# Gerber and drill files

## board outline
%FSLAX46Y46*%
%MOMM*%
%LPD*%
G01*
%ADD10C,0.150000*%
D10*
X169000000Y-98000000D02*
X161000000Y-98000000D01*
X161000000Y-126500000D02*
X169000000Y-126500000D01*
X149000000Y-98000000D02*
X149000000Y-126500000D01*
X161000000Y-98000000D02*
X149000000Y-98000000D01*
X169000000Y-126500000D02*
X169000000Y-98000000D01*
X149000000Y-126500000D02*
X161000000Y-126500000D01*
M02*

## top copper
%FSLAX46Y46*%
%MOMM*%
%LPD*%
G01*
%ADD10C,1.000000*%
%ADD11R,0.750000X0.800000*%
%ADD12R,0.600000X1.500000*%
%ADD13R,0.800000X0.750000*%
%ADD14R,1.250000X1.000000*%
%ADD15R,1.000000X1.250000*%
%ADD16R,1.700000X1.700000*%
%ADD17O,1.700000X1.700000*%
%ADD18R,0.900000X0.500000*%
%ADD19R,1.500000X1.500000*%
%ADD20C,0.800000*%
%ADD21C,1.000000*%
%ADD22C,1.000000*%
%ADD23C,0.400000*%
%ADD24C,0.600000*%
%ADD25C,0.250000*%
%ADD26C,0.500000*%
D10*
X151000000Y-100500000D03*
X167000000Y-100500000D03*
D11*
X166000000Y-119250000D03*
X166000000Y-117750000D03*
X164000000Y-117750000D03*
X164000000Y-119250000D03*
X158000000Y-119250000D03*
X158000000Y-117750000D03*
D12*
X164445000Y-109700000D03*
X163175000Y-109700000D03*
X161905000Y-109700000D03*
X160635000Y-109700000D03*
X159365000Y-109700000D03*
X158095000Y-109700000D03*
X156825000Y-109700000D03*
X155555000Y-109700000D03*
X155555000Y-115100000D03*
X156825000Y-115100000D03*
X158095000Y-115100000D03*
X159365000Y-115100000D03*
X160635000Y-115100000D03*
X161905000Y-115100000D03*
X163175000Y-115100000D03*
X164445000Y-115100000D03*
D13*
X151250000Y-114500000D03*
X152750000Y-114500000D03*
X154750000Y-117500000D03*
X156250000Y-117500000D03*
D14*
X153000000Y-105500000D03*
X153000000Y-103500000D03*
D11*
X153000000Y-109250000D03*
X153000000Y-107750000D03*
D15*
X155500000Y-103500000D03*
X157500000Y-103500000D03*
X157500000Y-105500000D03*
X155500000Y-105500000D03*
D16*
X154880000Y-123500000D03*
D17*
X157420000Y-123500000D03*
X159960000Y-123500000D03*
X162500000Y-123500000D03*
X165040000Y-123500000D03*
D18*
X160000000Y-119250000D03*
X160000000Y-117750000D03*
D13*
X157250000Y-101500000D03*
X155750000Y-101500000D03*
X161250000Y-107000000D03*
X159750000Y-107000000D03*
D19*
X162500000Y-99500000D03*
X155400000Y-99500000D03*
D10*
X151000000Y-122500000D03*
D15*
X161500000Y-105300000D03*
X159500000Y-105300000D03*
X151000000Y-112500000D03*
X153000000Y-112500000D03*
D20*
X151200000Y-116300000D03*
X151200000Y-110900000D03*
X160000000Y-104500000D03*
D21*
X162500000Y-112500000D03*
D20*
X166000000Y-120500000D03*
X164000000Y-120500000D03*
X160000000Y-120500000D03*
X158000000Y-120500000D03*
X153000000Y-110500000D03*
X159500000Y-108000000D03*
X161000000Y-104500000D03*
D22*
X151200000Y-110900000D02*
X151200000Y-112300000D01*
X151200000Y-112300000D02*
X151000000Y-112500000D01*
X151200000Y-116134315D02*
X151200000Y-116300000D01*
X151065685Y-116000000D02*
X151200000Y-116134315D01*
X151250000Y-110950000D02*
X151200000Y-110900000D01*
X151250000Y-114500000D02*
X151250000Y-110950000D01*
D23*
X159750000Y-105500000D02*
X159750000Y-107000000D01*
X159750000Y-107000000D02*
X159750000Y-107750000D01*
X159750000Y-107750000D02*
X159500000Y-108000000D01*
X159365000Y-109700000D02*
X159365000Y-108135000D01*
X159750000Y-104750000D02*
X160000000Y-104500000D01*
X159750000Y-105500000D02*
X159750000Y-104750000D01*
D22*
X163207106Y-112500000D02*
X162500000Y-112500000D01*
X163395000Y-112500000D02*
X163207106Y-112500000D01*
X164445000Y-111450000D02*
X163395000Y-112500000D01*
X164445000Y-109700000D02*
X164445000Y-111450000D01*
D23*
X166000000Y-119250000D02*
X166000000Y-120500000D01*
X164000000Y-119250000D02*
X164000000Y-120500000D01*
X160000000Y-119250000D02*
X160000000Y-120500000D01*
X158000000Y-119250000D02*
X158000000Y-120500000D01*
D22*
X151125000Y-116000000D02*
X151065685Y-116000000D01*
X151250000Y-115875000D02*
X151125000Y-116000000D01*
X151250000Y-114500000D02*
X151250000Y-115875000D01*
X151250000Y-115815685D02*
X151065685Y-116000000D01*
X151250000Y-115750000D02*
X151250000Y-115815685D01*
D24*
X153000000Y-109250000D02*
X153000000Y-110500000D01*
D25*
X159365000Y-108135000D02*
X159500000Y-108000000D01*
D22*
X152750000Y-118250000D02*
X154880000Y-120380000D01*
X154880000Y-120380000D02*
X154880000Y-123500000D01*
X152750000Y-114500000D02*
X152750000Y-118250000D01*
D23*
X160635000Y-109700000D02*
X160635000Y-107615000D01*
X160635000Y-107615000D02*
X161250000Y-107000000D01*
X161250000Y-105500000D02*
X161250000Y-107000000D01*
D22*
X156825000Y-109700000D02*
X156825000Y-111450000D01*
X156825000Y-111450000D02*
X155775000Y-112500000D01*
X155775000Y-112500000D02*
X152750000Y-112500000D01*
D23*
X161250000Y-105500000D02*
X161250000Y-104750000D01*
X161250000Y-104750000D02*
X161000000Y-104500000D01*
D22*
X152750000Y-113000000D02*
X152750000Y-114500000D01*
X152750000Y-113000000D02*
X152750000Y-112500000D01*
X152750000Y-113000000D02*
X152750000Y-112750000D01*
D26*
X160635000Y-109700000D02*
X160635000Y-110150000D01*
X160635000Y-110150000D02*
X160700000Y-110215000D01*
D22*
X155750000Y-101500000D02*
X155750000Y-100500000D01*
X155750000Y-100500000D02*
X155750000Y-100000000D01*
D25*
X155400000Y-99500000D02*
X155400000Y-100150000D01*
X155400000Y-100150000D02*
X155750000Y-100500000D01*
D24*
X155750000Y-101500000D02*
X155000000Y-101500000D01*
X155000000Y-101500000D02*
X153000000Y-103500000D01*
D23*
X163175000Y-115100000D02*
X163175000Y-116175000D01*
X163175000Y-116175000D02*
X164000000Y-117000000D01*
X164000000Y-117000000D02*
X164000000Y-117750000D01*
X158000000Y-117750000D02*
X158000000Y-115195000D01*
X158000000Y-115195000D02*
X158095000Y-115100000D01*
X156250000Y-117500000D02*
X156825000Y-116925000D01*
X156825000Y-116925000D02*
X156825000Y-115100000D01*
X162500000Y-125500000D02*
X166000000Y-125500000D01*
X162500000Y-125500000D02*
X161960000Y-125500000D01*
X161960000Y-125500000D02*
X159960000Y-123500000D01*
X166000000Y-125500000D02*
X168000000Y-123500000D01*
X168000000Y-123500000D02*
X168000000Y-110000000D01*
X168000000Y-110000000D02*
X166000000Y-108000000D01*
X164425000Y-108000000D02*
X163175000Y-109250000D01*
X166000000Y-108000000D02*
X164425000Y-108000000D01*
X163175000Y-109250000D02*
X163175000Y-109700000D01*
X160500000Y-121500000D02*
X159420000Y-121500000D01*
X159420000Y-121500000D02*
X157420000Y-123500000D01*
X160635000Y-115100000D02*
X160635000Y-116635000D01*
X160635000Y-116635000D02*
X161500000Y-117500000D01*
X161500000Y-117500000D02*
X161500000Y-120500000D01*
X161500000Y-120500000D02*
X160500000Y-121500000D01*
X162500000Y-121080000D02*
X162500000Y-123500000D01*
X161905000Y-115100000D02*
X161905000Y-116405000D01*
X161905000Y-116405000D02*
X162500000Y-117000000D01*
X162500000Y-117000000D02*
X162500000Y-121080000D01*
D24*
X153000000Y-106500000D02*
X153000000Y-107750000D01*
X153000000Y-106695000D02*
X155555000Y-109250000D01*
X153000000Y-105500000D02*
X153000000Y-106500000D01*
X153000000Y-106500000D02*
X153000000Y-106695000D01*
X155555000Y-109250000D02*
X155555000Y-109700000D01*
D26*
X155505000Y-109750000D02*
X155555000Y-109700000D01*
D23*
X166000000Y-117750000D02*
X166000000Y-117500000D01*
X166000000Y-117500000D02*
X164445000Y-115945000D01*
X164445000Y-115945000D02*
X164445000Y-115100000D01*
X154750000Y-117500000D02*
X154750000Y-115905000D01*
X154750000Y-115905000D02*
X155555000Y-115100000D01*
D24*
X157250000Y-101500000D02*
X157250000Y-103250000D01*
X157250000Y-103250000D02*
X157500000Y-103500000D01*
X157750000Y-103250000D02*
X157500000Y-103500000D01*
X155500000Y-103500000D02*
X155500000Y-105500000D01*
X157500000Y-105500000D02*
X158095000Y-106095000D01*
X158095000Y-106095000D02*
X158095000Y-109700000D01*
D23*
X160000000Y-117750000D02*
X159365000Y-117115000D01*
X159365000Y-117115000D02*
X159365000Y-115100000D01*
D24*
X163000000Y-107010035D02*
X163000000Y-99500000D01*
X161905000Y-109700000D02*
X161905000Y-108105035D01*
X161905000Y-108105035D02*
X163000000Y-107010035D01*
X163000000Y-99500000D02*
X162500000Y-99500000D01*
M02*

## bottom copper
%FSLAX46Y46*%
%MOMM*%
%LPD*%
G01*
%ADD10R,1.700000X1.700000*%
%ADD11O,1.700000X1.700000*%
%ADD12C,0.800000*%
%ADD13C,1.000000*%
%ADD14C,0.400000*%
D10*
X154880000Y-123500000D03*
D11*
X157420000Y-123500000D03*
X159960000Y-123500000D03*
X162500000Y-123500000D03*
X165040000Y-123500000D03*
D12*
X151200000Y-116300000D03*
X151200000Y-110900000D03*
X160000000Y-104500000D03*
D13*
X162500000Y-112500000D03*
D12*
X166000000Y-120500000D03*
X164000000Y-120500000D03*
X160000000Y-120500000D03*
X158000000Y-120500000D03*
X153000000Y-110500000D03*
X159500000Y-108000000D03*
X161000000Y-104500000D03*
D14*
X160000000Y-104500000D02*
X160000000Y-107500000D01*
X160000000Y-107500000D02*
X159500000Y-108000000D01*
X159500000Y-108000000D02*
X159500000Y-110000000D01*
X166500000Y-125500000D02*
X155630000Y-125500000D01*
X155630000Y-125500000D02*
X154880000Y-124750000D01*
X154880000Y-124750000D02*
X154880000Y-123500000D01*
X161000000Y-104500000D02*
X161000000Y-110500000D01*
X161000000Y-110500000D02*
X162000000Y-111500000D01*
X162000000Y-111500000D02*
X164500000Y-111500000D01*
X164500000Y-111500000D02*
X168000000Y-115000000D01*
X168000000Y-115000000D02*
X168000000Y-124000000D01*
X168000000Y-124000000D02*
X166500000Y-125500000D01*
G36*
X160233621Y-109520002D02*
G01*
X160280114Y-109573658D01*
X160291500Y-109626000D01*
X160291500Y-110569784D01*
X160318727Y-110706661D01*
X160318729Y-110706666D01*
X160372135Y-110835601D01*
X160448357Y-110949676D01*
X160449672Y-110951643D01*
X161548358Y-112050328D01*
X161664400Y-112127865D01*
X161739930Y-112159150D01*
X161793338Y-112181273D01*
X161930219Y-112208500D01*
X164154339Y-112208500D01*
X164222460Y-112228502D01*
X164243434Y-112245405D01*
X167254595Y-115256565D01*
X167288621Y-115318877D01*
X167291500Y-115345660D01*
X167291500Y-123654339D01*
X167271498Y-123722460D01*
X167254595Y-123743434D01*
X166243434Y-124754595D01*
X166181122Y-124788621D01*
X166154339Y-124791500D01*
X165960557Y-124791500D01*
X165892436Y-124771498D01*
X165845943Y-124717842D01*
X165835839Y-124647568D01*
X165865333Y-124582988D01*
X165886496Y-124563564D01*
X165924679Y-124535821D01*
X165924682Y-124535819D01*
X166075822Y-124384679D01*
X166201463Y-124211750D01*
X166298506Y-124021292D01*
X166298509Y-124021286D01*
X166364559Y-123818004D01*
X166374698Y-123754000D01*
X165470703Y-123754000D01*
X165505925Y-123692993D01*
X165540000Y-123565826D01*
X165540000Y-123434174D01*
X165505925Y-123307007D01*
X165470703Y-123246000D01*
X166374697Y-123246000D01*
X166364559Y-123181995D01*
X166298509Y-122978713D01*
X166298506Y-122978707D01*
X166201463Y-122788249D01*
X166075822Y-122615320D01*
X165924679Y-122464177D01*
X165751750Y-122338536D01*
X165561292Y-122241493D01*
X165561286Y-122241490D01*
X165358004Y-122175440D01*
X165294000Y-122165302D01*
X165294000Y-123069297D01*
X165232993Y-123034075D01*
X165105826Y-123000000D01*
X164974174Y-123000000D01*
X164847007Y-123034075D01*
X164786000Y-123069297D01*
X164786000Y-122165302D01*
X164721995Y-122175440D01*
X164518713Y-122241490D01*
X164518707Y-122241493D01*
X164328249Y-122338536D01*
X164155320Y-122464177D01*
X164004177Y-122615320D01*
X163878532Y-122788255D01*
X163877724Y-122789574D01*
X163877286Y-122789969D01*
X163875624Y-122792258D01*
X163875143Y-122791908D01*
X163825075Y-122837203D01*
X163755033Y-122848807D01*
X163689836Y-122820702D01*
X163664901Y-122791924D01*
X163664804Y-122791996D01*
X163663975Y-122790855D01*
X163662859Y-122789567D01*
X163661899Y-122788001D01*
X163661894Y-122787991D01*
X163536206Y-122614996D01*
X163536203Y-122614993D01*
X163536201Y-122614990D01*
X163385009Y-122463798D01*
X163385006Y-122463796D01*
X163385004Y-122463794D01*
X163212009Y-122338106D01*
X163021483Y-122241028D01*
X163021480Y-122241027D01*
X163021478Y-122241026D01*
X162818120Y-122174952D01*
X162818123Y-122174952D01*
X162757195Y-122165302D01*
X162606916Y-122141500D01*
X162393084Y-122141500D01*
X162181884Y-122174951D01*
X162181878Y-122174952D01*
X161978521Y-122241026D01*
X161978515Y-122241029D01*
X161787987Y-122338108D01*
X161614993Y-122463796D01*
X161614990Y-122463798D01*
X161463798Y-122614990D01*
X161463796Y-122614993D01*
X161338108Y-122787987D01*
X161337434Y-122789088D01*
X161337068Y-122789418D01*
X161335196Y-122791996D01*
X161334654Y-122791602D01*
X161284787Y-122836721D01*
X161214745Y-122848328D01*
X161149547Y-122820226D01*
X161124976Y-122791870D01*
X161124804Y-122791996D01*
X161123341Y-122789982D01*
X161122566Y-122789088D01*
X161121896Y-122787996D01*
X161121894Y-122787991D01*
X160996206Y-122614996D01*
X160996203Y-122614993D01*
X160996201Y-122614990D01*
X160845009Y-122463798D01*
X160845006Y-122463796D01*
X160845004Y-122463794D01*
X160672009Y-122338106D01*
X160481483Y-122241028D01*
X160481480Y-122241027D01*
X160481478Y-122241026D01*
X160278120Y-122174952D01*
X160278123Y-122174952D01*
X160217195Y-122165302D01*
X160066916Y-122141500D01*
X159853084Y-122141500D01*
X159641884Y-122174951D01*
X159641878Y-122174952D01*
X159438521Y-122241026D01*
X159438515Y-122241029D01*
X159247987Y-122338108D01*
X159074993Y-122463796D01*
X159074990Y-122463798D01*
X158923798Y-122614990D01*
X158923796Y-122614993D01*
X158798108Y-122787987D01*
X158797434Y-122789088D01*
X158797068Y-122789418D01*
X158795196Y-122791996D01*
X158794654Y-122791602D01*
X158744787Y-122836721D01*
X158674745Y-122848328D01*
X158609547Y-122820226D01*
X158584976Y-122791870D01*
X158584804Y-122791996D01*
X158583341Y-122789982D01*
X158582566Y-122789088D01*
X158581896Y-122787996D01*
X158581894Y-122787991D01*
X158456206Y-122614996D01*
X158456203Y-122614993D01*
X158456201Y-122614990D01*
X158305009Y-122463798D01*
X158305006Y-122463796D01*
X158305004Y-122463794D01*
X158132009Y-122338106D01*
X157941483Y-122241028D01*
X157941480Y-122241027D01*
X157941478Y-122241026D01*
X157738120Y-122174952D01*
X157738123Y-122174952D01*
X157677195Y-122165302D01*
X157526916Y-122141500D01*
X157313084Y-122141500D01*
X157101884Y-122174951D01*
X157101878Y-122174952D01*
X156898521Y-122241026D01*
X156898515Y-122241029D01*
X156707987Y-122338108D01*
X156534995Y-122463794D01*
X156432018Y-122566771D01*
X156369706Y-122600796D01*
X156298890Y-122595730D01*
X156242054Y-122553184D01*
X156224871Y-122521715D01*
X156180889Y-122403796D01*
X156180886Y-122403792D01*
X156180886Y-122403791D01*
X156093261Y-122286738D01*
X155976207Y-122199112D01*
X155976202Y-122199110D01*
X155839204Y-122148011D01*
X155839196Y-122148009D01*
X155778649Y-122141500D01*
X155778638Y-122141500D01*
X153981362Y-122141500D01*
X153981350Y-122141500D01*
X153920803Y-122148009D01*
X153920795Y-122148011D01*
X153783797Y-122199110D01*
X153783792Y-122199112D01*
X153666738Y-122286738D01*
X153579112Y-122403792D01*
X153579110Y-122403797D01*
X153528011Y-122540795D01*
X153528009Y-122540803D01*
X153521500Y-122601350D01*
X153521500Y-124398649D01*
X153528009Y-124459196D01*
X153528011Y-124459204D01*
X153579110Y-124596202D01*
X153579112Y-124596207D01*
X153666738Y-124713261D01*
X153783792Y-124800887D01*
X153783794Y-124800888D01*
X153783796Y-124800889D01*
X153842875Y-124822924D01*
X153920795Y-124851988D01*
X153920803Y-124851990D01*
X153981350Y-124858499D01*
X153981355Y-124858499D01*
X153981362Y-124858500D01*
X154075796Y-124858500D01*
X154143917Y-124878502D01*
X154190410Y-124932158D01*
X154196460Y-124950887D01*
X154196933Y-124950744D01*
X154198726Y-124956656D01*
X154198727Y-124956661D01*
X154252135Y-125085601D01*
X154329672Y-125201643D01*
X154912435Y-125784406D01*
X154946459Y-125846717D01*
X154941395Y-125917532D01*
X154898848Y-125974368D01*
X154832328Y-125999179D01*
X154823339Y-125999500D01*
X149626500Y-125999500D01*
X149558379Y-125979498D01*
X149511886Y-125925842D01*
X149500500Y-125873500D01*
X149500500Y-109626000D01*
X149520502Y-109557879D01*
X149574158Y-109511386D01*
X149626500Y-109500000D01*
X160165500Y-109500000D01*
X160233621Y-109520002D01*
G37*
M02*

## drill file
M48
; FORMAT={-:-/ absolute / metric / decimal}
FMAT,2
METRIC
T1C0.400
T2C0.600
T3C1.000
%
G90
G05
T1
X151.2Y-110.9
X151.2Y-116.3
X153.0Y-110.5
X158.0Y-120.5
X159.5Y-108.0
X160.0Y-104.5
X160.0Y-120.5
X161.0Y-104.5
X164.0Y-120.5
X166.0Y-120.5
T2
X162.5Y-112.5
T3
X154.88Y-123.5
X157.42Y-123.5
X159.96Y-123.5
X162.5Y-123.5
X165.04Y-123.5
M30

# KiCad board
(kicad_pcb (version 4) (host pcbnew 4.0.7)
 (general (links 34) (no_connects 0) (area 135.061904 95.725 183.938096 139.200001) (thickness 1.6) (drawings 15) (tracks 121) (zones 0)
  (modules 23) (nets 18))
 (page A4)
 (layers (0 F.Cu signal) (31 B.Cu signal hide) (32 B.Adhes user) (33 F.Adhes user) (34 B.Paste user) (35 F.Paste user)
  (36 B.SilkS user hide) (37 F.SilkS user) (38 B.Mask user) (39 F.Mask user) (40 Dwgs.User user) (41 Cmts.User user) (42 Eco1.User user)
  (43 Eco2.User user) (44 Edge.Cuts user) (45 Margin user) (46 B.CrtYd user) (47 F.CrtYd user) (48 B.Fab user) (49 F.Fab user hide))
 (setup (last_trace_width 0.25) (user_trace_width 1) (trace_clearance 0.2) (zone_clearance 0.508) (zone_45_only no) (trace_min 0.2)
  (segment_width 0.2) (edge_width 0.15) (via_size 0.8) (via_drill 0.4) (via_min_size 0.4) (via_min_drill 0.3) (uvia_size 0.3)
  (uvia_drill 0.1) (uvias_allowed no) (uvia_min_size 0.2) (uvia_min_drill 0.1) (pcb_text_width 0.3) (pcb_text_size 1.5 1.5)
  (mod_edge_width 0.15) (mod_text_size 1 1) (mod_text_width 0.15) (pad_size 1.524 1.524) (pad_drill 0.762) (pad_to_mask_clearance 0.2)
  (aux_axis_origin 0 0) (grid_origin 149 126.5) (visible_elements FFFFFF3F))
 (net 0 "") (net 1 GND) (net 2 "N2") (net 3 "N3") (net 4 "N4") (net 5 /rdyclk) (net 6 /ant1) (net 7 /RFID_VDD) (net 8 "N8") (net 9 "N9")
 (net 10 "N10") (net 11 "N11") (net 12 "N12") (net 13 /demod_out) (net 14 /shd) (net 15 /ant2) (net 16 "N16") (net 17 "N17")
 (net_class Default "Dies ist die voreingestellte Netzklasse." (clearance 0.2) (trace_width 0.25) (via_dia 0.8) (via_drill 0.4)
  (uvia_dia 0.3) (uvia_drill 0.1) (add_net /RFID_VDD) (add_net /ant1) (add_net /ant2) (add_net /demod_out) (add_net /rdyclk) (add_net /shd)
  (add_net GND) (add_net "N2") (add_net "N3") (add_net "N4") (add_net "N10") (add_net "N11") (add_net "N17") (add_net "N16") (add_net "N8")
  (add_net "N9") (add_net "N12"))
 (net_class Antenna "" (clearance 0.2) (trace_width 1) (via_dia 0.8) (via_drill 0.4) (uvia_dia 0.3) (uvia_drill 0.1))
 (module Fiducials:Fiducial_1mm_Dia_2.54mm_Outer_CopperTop (layer F.Cu) (at 151 100.5)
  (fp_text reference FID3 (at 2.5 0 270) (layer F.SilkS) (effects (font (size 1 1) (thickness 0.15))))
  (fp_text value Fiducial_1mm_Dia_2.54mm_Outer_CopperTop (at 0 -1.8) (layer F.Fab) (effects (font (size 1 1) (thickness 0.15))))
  (pad ~ smd circle (at 0 0) (size 1 1) (layers F.Cu F.Mask) (solder_mask_margin 0.77) (clearance 0.77)))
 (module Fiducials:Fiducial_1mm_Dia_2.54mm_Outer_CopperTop (layer F.Cu) (at 167 100.5)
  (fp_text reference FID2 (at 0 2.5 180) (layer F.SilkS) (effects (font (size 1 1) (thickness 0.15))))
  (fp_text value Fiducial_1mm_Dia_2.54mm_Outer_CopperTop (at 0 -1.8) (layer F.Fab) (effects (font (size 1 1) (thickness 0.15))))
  (pad ~ smd circle (at 0 0) (size 1 1) (layers F.Cu F.Mask) (solder_mask_margin 0.77) (clearance 0.77)))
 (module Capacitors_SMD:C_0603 (layer F.Cu) (at 166 118.5 90)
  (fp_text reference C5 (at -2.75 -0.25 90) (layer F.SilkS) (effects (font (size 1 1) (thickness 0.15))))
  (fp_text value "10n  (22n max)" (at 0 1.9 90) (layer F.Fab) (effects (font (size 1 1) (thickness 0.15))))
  (pad 1 smd rect (at -0.75 0 90) (size 0.8 0.75) (layers F.Cu F.Paste F.Mask) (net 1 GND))
  (pad 2 smd rect (at 0.75 0 90) (size 0.8 0.75) (layers F.Cu F.Paste F.Mask) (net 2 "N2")))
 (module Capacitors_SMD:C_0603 (layer F.Cu) (at 164 118.5 90)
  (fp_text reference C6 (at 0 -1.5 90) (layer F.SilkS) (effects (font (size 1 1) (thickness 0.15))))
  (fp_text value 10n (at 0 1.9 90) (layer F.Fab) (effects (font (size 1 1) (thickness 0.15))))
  (pad 2 smd rect (at 0.75 0 90) (size 0.8 0.75) (layers F.Cu F.Paste F.Mask) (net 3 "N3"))
  (pad 1 smd rect (at -0.75 0 90) (size 0.8 0.75) (layers F.Cu F.Paste F.Mask) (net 1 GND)))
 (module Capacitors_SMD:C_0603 (layer F.Cu) (at 158 118.5 90)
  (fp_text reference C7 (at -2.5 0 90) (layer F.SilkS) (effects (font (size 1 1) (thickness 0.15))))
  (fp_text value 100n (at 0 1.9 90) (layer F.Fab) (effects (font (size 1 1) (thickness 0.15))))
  (pad 1 smd rect (at -0.75 0 90) (size 0.8 0.75) (layers F.Cu F.Paste F.Mask) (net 1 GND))
  (pad 2 smd rect (at 0.75 0 90) (size 0.8 0.75) (layers F.Cu F.Paste F.Mask) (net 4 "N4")))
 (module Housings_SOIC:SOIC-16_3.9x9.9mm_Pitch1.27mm (layer F.Cu) (at 160 112.4 270)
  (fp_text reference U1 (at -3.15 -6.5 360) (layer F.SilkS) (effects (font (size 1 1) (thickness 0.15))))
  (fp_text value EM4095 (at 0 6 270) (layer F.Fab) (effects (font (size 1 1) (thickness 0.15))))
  (pad 1 smd rect (at -2.7 -4.445 270) (size 1.5 0.6) (layers F.Cu F.Paste F.Mask) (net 1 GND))
  (pad 2 smd rect (at -2.7 -3.175 270) (size 1.5 0.6) (layers F.Cu F.Paste F.Mask) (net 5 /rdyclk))
  (pad 3 smd rect (at -2.7 -1.905 270) (size 1.5 0.6) (layers F.Cu F.Paste F.Mask) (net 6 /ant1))
  (pad 4 smd rect (at -2.7 -0.635 270) (size 1.5 0.6) (layers F.Cu F.Paste F.Mask) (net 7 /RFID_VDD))
  (pad 5 smd rect (at -2.7 0.635 270) (size 1.5 0.6) (layers F.Cu F.Paste F.Mask) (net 1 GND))
  (pad 6 smd rect (at -2.7 1.905 270) (size 1.5 0.6) (layers F.Cu F.Paste F.Mask) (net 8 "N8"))
  (pad 7 smd rect (at -2.7 3.175 270) (size 1.5 0.6) (layers F.Cu F.Paste F.Mask) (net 7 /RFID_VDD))
  (pad 8 smd rect (at -2.7 4.445 270) (size 1.5 0.6) (layers F.Cu F.Paste F.Mask) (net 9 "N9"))
  (pad 9 smd rect (at 2.7 4.445 270) (size 1.5 0.6) (layers F.Cu F.Paste F.Mask) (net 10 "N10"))
  (pad 10 smd rect (at 2.7 3.175 270) (size 1.5 0.6) (layers F.Cu F.Paste F.Mask) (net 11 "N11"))
  (pad 11 smd rect (at 2.7 1.905 270) (size 1.5 0.6) (layers F.Cu F.Paste F.Mask) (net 4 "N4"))
  (pad 12 smd rect (at 2.7 0.635 270) (size 1.5 0.6) (layers F.Cu F.Paste F.Mask) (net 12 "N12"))
  (pad 13 smd rect (at 2.7 -0.635 270) (size 1.5 0.6) (layers F.Cu F.Paste F.Mask) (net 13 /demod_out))
  (pad 14 smd rect (at 2.7 -1.905 270) (size 1.5 0.6) (layers F.Cu F.Paste F.Mask) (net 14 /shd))
  (pad 15 smd rect (at 2.7 -3.175 270) (size 1.5 0.6) (layers F.Cu F.Paste F.Mask) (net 3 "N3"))
  (pad 16 smd rect (at 2.7 -4.445 270) (size 1.5 0.6) (layers F.Cu F.Paste F.Mask) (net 2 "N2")))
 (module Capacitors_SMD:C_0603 (layer F.Cu) (at 152 114.5)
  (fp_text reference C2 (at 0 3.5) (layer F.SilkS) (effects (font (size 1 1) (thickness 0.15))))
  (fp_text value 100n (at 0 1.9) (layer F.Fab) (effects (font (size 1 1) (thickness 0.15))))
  (pad 1 smd rect (at -0.75 0) (size 0.8 0.75) (layers F.Cu F.Paste F.Mask) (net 1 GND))
  (pad 2 smd rect (at 0.75 0) (size 0.8 0.75) (layers F.Cu F.Paste F.Mask) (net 7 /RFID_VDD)))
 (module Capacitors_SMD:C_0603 (layer F.Cu) (at 155.5 117.5)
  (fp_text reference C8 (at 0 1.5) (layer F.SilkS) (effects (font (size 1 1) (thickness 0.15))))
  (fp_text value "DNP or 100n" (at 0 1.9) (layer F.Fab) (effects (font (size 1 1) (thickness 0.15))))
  (pad 1 smd rect (at -0.75 0) (size 0.8 0.75) (layers F.Cu F.Paste F.Mask) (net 10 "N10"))
  (pad 2 smd rect (at 0.75 0) (size 0.8 0.75) (layers F.Cu F.Paste F.Mask) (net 11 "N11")))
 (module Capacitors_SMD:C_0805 (layer F.Cu) (at 153 104.5 90)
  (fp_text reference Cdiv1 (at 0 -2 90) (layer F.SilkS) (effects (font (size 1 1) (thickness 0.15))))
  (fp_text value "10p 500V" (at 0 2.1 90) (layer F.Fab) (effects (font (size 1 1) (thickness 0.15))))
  (pad 1 smd rect (at -1 0 90) (size 1 1.25) (layers F.Cu F.Paste F.Mask) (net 9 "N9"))
  (pad 2 smd rect (at 1 0 90) (size 1 1.25) (layers F.Cu F.Paste F.Mask) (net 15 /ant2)))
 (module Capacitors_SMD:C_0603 (layer F.Cu) (at 153 108.5 90)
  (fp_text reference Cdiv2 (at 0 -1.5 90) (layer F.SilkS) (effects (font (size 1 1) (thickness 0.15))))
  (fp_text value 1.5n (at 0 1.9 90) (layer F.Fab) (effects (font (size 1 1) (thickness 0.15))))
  (pad 1 smd rect (at -0.75 0 90) (size 0.8 0.75) (layers F.Cu F.Paste F.Mask) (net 1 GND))
  (pad 2 smd rect (at 0.75 0 90) (size 0.8 0.75) (layers F.Cu F.Paste F.Mask) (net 9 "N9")))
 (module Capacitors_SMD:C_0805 (layer F.Cu) (at 156.5 103.5)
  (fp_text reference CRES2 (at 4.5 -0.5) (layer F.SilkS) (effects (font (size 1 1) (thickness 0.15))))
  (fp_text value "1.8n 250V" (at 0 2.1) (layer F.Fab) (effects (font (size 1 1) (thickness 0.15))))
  (pad 1 smd rect (at -1 0) (size 1 1.25) (layers F.Cu F.Paste F.Mask) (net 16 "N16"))
  (pad 2 smd rect (at 1 0) (size 1 1.25) (layers F.Cu F.Paste F.Mask) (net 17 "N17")))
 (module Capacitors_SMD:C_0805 (layer F.Cu) (at 156.5 105.5 180)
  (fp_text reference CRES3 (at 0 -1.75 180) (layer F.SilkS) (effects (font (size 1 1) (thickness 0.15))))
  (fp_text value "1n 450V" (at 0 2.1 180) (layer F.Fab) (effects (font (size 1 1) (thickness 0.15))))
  (pad 1 smd rect (at -1 0 180) (size 1 1.25) (layers F.Cu F.Paste F.Mask) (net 8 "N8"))
  (pad 2 smd rect (at 1 0 180) (size 1 1.25) (layers F.Cu F.Paste F.Mask) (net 16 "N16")))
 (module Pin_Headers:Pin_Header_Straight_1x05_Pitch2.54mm (layer F.Cu) (at 154.88 123.5 90)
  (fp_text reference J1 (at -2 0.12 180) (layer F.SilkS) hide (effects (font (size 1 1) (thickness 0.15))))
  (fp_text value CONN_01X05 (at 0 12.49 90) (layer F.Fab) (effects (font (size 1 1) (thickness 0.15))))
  (pad 1 thru_hole rect (at 0 0 90) (size 1.7 1.7) (drill 1) (layers *.Cu *.Mask) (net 7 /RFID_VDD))
  (pad 2 thru_hole oval (at 0 2.54 90) (size 1.7 1.7) (drill 1) (layers *.Cu *.Mask) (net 13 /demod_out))
  (pad 3 thru_hole oval (at 0 5.08 90) (size 1.7 1.7) (drill 1) (layers *.Cu *.Mask) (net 5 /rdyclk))
  (pad 4 thru_hole oval (at 0 7.62 90) (size 1.7 1.7) (drill 1) (layers *.Cu *.Mask) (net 14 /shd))
  (pad 5 thru_hole oval (at 0 10.16 90) (size 1.7 1.7) (drill 1) (layers *.Cu *.Mask) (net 1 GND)))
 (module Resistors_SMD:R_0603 (layer F.Cu) (at 160 118.5 90)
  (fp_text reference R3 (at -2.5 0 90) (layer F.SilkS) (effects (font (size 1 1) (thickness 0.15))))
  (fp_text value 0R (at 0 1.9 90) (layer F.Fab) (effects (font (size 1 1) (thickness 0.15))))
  (pad 1 smd rect (at -0.75 0 90) (size 0.5 0.9) (layers F.Cu F.Paste F.Mask) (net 1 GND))
  (pad 2 smd rect (at 0.75 0 90) (size 0.5 0.9) (layers F.Cu F.Paste F.Mask) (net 12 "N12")))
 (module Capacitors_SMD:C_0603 (layer F.Cu) (at 156.5 101.5 180)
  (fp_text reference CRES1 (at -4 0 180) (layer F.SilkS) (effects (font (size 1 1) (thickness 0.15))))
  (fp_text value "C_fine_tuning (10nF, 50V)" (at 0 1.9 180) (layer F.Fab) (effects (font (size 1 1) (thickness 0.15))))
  (pad 1 smd rect (at -0.75 0 180) (size 0.8 0.75) (layers F.Cu F.Paste F.Mask) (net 17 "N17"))
  (pad 2 smd rect (at 0.75 0 180) (size 0.8 0.75) (layers F.Cu F.Paste F.Mask) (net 15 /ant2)))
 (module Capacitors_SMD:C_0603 (layer F.Cu) (at 160.5 107 180)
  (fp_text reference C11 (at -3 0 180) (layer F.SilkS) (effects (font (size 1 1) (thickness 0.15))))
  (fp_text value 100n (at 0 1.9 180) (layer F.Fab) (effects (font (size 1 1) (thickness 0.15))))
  (pad 1 smd rect (at -0.75 0 180) (size 0.8 0.75) (layers F.Cu F.Paste F.Mask) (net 7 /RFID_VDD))
  (pad 2 smd rect (at 0.75 0 180) (size 0.8 0.75) (layers F.Cu F.Paste F.Mask) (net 1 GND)))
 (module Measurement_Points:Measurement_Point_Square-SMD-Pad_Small (layer F.Cu) (at 162.5 99.5)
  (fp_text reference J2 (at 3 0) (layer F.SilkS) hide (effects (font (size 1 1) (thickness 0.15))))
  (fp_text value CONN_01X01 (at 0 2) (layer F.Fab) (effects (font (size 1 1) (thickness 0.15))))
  (pad 1 smd rect (at 0 0) (size 1.5 1.5) (layers F.Cu F.Mask) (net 6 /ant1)))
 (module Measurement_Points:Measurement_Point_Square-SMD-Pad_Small (layer F.Cu) (at 155.4 99.5)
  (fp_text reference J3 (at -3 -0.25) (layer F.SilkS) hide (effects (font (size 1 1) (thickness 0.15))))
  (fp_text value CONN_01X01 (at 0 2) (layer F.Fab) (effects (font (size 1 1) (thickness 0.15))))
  (pad 1 smd rect (at 0 0) (size 1.5 1.5) (layers F.Cu F.Mask) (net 15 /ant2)))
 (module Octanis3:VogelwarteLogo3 (layer B.Cu) (at 159 119 180)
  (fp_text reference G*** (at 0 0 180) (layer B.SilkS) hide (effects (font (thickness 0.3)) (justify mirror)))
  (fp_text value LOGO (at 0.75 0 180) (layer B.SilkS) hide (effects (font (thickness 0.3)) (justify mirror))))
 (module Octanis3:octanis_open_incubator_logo (layer B.Cu) (at 159 106.5 180)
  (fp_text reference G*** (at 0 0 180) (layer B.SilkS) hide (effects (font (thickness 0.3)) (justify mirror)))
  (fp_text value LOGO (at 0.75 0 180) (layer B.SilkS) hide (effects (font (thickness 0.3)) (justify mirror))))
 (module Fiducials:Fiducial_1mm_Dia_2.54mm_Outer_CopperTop (layer F.Cu) (at 151 122.5)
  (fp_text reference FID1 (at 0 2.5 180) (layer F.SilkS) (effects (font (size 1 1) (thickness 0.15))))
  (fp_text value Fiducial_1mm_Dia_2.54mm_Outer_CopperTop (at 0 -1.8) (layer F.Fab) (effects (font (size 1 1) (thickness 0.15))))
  (pad ~ smd circle (at 0 0) (size 1 1) (layers F.Cu F.Mask) (solder_mask_margin 0.77) (clearance 0.77)))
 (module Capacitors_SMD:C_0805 (layer F.Cu) (at 160.5 105.3 180)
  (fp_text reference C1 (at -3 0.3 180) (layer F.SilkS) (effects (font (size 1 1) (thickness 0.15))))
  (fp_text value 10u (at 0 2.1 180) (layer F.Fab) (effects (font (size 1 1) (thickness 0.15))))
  (pad 1 smd rect (at -1 0 180) (size 1 1.25) (layers F.Cu F.Paste F.Mask) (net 7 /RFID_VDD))
  (pad 2 smd rect (at 1 0 180) (size 1 1.25) (layers F.Cu F.Paste F.Mask) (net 1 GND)))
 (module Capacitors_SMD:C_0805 (layer F.Cu) (at 152 112.5)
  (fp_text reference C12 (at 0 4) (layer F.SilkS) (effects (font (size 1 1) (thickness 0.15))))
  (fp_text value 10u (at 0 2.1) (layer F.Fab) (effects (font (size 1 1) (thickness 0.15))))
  (pad 1 smd rect (at -1 0) (size 1 1.25) (layers F.Cu F.Paste F.Mask) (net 1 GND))
  (pad 2 smd rect (at 1 0) (size 1 1.25) (layers F.Cu F.Paste F.Mask) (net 7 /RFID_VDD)))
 (gr_line (start 169 98) (end 161 98) (layer Edge.Cuts) (width 0.15))
 (gr_line (start 161 126.5) (end 169 126.5) (layer Edge.Cuts) (width 0.15))
 (gr_line (start 149 98) (end 149 126.5) (layer Edge.Cuts) (width 0.15))
 (gr_line (start 161 98) (end 149 98) (layer Edge.Cuts) (width 0.15))
 (gr_line (start 169 126.5) (end 169 98) (layer Edge.Cuts) (width 0.15))
 (gr_line (start 149 126.5) (end 161 126.5) (layer Edge.Cuts) (width 0.15))
 (segment (start 151.2 110.9) (end 151.2 112.3) (width 1) (layer F.Cu) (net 1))
 (segment (start 151.2 112.3) (end 151 112.5) (width 1) (layer F.Cu) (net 1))
 (segment (start 151.2 116.134315) (end 151.2 116.3) (width 1) (layer F.Cu) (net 1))
 (segment (start 151.065685 116) (end 151.2 116.134315) (width 1) (layer F.Cu) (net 1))
 (via (at 151.2 116.3) (size 0.8) (drill 0.4) (layers F.Cu B.Cu) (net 1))
 (segment (start 151.25 110.95) (end 151.2 110.9) (width 1) (layer F.Cu) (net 1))
 (segment (start 151.25 114.5) (end 151.25 110.95) (width 1) (layer F.Cu) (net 1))
 (via (at 151.2 110.9) (size 0.8) (drill 0.4) (layers F.Cu B.Cu) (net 1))
 (segment (start 159.75 105.5) (end 159.75 107) (width 0.4) (layer F.Cu) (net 1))
 (segment (start 159.75 107) (end 159.75 107.75) (width 0.4) (layer F.Cu) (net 1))
 (segment (start 159.75 107.75) (end 159.5 108) (width 0.4) (layer F.Cu) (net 1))
 (segment (start 159.365 109.7) (end 159.365 108.135) (width 0.4) (layer F.Cu) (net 1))
 (segment (start 159.75 104.75) (end 160 104.5) (width 0.4) (layer F.Cu) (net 1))
 (segment (start 159.75 105.5) (end 159.75 104.75) (width 0.4) (layer F.Cu) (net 1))
 (segment (start 160 104.5) (end 160 107.5) (width 0.4) (layer B.Cu) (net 1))
 (segment (start 160 107.5) (end 159.5 108) (width 0.4) (layer B.Cu) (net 1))
 (via (at 160 104.5) (size 0.8) (drill 0.4) (layers F.Cu B.Cu) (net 1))
 (segment (start 159.5 108) (end 159.5 110) (width 0.4) (layer B.Cu) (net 1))
 (segment (start 163.207106 112.5) (end 162.5 112.5) (width 1) (layer F.Cu) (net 1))
 (segment (start 163.395 112.5) (end 163.207106 112.5) (width 1) (layer F.Cu) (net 1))
 (segment (start 164.445 111.45) (end 163.395 112.5) (width 1) (layer F.Cu) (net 1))
 (segment (start 164.445 109.7) (end 164.445 111.45) (width 1) (layer F.Cu) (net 1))
 (via (at 162.5 112.5) (size 1) (drill 0.6) (layers F.Cu B.Cu) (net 1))
 (segment (start 166 119.25) (end 166 120.5) (width 0.4) (layer F.Cu) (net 1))
 (via (at 166 120.5) (size 0.8) (drill 0.4) (layers F.Cu B.Cu) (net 1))
 (segment (start 164 119.25) (end 164 120.5) (width 0.4) (layer F.Cu) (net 1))
 (via (at 164 120.5) (size 0.8) (drill 0.4) (layers F.Cu B.Cu) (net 1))
 (segment (start 160 119.25) (end 160 120.5) (width 0.4) (layer F.Cu) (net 1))
 (via (at 160 120.5) (size 0.8) (drill 0.4) (layers F.Cu B.Cu) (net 1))
 (segment (start 158 119.25) (end 158 120.5) (width 0.4) (layer F.Cu) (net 1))
 (via (at 158 120.5) (size 0.8) (drill 0.4) (layers F.Cu B.Cu) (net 1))
 (segment (start 151.125 116) (end 151.065685 116) (width 1) (layer F.Cu) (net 1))
 (segment (start 151.25 115.875) (end 151.125 116) (width 1) (layer F.Cu) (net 1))
 (segment (start 151.25 114.5) (end 151.25 115.875) (width 1) (layer F.Cu) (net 1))
 (segment (start 151.25 115.815685) (end 151.065685 116) (width 1) (layer F.Cu) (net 1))
 (segment (start 151.25 115.75) (end 151.25 115.815685) (width 1) (layer F.Cu) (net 1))
 (segment (start 153 109.25) (end 153 110.5) (width 0.6) (layer F.Cu) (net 1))
 (via (at 153 110.5) (size 0.8) (drill 0.4) (layers F.Cu B.Cu) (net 1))
 (via (at 159.5 108) (size 0.8) (drill 0.4) (layers F.Cu B.Cu) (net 1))
 (segment (start 159.365 108.135) (end 159.5 108) (width 0.25) (layer F.Cu) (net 1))
 (segment (start 166.5 125.5) (end 155.63 125.5) (width 0.4) (layer B.Cu) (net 7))
 (segment (start 155.63 125.5) (end 154.88 124.75) (width 0.4) (layer B.Cu) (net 7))
 (segment (start 154.88 124.75) (end 154.88 123.5) (width 0.4) (layer B.Cu) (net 7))
 (segment (start 152.75 118.25) (end 154.88 120.38) (width 1) (layer F.Cu) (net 7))
 (segment (start 154.88 120.38) (end 154.88 123.5) (width 1) (layer F.Cu) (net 7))
 (segment (start 152.75 114.5) (end 152.75 118.25) (width 1) (layer F.Cu) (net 7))
 (segment (start 161 104.5) (end 161 110.5) (width 0.4) (layer B.Cu) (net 7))
 (segment (start 161 110.5) (end 162 111.5) (width 0.4) (layer B.Cu) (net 7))
 (segment (start 162 111.5) (end 164.5 111.5) (width 0.4) (layer B.Cu) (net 7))
 (segment (start 164.5 111.5) (end 168 115) (width 0.4) (layer B.Cu) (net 7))
 (segment (start 168 115) (end 168 124) (width 0.4) (layer B.Cu) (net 7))
 (segment (start 168 124) (end 166.5 125.5) (width 0.4) (layer B.Cu) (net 7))
 (segment (start 160.635 109.7) (end 160.635 107.615) (width 0.4) (layer F.Cu) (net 7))
 (segment (start 160.635 107.615) (end 161.25 107) (width 0.4) (layer F.Cu) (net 7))
 (segment (start 161.25 105.5) (end 161.25 107) (width 0.4) (layer F.Cu) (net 7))
 (segment (start 156.825 109.7) (end 156.825 111.45) (width 1) (layer F.Cu) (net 7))
 (segment (start 156.825 111.45) (end 155.775 112.5) (width 1) (layer F.Cu) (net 7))
 (segment (start 155.775 112.5) (end 152.75 112.5) (width 1) (layer F.Cu) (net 7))
 (segment (start 161.25 105.5) (end 161.25 104.75) (width 0.4) (layer F.Cu) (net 7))
 (segment (start 161.25 104.75) (end 161 104.5) (width 0.4) (layer F.Cu) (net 7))
 (via (at 161 104.5) (size 0.8) (drill 0.4) (layers F.Cu B.Cu) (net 7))
 (segment (start 152.75 113) (end 152.75 114.5) (width 1) (layer F.Cu) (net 7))
 (segment (start 152.75 113) (end 152.75 112.5) (width 1) (layer F.Cu) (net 7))
 (segment (start 152.75 113) (end 152.75 112.75) (width 1) (layer F.Cu) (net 7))
 (segment (start 160.635 109.7) (end 160.635 110.15) (width 0.5) (layer F.Cu) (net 7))
 (segment (start 160.635 110.15) (end 160.7 110.215) (width 0.5) (layer F.Cu) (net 7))
 (segment (start 155.75 101.5) (end 155.75 100.5) (width 1) (layer F.Cu) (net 15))
 (segment (start 155.75 100.5) (end 155.75 100) (width 1) (layer F.Cu) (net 15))
 (segment (start 155.4 99.5) (end 155.4 100.15) (width 0.25) (layer F.Cu) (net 15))
 (segment (start 155.4 100.15) (end 155.75 100.5) (width 0.25) (layer F.Cu) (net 15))
 (segment (start 155.75 101.5) (end 155 101.5) (width 0.6) (layer F.Cu) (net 15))
 (segment (start 155 101.5) (end 153 103.5) (width 0.6) (layer F.Cu) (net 15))
 (segment (start 163.175 115.1) (end 163.175 116.175) (width 0.4) (layer F.Cu) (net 3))
 (segment (start 163.175 116.175) (end 164 117) (width 0.4) (layer F.Cu) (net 3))
 (segment (start 164 117) (end 164 117.75) (width 0.4) (layer F.Cu) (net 3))
 (segment (start 158 117.75) (end 158 115.195) (width 0.4) (layer F.Cu) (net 4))
 (segment (start 158 115.195) (end 158.095 115.1) (width 0.4) (layer F.Cu) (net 4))
 (segment (start 156.25 117.5) (end 156.825 116.925) (width 0.4) (layer F.Cu) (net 11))
 (segment (start 156.825 116.925) (end 156.825 115.1) (width 0.4) (layer F.Cu) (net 11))
 (segment (start 162.5 125.5) (end 166 125.5) (width 0.4) (layer F.Cu) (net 5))
 (segment (start 162.5 125.5) (end 161.96 125.5) (width 0.4) (layer F.Cu) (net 5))
 (segment (start 161.96 125.5) (end 159.96 123.5) (width 0.4) (layer F.Cu) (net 5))
 (segment (start 166 125.5) (end 168 123.5) (width 0.4) (layer F.Cu) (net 5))
 (segment (start 168 123.5) (end 168 110) (width 0.4) (layer F.Cu) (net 5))
 (segment (start 168 110) (end 166 108) (width 0.4) (layer F.Cu) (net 5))
 (segment (start 164.425 108) (end 163.175 109.25) (width 0.4) (layer F.Cu) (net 5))
 (segment (start 166 108) (end 164.425 108) (width 0.4) (layer F.Cu) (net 5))
 (segment (start 163.175 109.25) (end 163.175 109.7) (width 0.4) (layer F.Cu) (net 5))
 (segment (start 160.5 121.5) (end 159.42 121.5) (width 0.4) (layer F.Cu) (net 13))
 (segment (start 159.42 121.5) (end 157.42 123.5) (width 0.4) (layer F.Cu) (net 13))
 (segment (start 160.635 115.1) (end 160.635 116.635) (width 0.4) (layer F.Cu) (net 13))
 (segment (start 160.635 116.635) (end 161.5 117.5) (width 0.4) (layer F.Cu) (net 13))
 (segment (start 161.5 117.5) (end 161.5 120.5) (width 0.4) (layer F.Cu) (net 13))
 (segment (start 161.5 120.5) (end 160.5 121.5) (width 0.4) (layer F.Cu) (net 13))
 (segment (start 162.5 121.08) (end 162.5 123.5) (width 0.4) (layer F.Cu) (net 14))
 (segment (start 161.905 115.1) (end 161.905 116.405) (width 0.4) (layer F.Cu) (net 14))
 (segment (start 161.905 116.405) (end 162.5 117) (width 0.4) (layer F.Cu) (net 14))
 (segment (start 162.5 117) (end 162.5 121.08) (width 0.4) (layer F.Cu) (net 14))
 (segment (start 153 106.5) (end 153 107.75) (width 0.6) (layer F.Cu) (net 9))
 (segment (start 153 106.695) (end 155.555 109.25) (width 0.6) (layer F.Cu) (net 9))
 (segment (start 153 105.5) (end 153 106.5) (width 0.6) (layer F.Cu) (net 9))
 (segment (start 153 106.5) (end 153 106.695) (width 0.6) (layer F.Cu) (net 9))
 (segment (start 155.555 109.25) (end 155.555 109.7) (width 0.6) (layer F.Cu) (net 9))
 (segment (start 155.505 109.75) (end 155.555 109.7) (width 0.5) (layer F.Cu) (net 9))
 (segment (start 166 117.75) (end 166 117.5) (width 0.4) (layer F.Cu) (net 2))
 (segment (start 166 117.5) (end 164.445 115.945) (width 0.4) (layer F.Cu) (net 2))
 (segment (start 164.445 115.945) (end 164.445 115.1) (width 0.4) (layer F.Cu) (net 2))
 (segment (start 154.75 117.5) (end 154.75 115.905) (width 0.4) (layer F.Cu) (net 10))
 (segment (start 154.75 115.905) (end 155.555 115.1) (width 0.4) (layer F.Cu) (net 10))
 (segment (start 157.25 101.5) (end 157.25 103.25) (width 0.6) (layer F.Cu) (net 17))
 (segment (start 157.25 103.25) (end 157.5 103.5) (width 0.6) (layer F.Cu) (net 17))
 (segment (start 157.75 103.25) (end 157.5 103.5) (width 0.6) (layer F.Cu) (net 17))
 (segment (start 155.5 103.5) (end 155.5 105.5) (width 0.6) (layer F.Cu) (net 16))
 (segment (start 157.5 105.5) (end 158.095 106.095) (width 0.6) (layer F.Cu) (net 8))
 (segment (start 158.095 106.095) (end 158.095 109.7) (width 0.6) (layer F.Cu) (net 8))
 (segment (start 160 117.75) (end 159.365 117.115) (width 0.4) (layer F.Cu) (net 12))
 (segment (start 159.365 117.115) (end 159.365 115.1) (width 0.4) (layer F.Cu) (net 12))
 (segment (start 163 107.010035) (end 163 99.5) (width 0.6) (layer F.Cu) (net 6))
 (segment (start 161.905 109.7) (end 161.905 108.105035) (width 0.6) (layer F.Cu) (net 6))
 (segment (start 161.905 108.105035) (end 163 107.010035) (width 0.6) (layer F.Cu) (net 6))
 (segment (start 163 99.5) (end 162.5 99.5) (width 0.6) (layer F.Cu) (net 6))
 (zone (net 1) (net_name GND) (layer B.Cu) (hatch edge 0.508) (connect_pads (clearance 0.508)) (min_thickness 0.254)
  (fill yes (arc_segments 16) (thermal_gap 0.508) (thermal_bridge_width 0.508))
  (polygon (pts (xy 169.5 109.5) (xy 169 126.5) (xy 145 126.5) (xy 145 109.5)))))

